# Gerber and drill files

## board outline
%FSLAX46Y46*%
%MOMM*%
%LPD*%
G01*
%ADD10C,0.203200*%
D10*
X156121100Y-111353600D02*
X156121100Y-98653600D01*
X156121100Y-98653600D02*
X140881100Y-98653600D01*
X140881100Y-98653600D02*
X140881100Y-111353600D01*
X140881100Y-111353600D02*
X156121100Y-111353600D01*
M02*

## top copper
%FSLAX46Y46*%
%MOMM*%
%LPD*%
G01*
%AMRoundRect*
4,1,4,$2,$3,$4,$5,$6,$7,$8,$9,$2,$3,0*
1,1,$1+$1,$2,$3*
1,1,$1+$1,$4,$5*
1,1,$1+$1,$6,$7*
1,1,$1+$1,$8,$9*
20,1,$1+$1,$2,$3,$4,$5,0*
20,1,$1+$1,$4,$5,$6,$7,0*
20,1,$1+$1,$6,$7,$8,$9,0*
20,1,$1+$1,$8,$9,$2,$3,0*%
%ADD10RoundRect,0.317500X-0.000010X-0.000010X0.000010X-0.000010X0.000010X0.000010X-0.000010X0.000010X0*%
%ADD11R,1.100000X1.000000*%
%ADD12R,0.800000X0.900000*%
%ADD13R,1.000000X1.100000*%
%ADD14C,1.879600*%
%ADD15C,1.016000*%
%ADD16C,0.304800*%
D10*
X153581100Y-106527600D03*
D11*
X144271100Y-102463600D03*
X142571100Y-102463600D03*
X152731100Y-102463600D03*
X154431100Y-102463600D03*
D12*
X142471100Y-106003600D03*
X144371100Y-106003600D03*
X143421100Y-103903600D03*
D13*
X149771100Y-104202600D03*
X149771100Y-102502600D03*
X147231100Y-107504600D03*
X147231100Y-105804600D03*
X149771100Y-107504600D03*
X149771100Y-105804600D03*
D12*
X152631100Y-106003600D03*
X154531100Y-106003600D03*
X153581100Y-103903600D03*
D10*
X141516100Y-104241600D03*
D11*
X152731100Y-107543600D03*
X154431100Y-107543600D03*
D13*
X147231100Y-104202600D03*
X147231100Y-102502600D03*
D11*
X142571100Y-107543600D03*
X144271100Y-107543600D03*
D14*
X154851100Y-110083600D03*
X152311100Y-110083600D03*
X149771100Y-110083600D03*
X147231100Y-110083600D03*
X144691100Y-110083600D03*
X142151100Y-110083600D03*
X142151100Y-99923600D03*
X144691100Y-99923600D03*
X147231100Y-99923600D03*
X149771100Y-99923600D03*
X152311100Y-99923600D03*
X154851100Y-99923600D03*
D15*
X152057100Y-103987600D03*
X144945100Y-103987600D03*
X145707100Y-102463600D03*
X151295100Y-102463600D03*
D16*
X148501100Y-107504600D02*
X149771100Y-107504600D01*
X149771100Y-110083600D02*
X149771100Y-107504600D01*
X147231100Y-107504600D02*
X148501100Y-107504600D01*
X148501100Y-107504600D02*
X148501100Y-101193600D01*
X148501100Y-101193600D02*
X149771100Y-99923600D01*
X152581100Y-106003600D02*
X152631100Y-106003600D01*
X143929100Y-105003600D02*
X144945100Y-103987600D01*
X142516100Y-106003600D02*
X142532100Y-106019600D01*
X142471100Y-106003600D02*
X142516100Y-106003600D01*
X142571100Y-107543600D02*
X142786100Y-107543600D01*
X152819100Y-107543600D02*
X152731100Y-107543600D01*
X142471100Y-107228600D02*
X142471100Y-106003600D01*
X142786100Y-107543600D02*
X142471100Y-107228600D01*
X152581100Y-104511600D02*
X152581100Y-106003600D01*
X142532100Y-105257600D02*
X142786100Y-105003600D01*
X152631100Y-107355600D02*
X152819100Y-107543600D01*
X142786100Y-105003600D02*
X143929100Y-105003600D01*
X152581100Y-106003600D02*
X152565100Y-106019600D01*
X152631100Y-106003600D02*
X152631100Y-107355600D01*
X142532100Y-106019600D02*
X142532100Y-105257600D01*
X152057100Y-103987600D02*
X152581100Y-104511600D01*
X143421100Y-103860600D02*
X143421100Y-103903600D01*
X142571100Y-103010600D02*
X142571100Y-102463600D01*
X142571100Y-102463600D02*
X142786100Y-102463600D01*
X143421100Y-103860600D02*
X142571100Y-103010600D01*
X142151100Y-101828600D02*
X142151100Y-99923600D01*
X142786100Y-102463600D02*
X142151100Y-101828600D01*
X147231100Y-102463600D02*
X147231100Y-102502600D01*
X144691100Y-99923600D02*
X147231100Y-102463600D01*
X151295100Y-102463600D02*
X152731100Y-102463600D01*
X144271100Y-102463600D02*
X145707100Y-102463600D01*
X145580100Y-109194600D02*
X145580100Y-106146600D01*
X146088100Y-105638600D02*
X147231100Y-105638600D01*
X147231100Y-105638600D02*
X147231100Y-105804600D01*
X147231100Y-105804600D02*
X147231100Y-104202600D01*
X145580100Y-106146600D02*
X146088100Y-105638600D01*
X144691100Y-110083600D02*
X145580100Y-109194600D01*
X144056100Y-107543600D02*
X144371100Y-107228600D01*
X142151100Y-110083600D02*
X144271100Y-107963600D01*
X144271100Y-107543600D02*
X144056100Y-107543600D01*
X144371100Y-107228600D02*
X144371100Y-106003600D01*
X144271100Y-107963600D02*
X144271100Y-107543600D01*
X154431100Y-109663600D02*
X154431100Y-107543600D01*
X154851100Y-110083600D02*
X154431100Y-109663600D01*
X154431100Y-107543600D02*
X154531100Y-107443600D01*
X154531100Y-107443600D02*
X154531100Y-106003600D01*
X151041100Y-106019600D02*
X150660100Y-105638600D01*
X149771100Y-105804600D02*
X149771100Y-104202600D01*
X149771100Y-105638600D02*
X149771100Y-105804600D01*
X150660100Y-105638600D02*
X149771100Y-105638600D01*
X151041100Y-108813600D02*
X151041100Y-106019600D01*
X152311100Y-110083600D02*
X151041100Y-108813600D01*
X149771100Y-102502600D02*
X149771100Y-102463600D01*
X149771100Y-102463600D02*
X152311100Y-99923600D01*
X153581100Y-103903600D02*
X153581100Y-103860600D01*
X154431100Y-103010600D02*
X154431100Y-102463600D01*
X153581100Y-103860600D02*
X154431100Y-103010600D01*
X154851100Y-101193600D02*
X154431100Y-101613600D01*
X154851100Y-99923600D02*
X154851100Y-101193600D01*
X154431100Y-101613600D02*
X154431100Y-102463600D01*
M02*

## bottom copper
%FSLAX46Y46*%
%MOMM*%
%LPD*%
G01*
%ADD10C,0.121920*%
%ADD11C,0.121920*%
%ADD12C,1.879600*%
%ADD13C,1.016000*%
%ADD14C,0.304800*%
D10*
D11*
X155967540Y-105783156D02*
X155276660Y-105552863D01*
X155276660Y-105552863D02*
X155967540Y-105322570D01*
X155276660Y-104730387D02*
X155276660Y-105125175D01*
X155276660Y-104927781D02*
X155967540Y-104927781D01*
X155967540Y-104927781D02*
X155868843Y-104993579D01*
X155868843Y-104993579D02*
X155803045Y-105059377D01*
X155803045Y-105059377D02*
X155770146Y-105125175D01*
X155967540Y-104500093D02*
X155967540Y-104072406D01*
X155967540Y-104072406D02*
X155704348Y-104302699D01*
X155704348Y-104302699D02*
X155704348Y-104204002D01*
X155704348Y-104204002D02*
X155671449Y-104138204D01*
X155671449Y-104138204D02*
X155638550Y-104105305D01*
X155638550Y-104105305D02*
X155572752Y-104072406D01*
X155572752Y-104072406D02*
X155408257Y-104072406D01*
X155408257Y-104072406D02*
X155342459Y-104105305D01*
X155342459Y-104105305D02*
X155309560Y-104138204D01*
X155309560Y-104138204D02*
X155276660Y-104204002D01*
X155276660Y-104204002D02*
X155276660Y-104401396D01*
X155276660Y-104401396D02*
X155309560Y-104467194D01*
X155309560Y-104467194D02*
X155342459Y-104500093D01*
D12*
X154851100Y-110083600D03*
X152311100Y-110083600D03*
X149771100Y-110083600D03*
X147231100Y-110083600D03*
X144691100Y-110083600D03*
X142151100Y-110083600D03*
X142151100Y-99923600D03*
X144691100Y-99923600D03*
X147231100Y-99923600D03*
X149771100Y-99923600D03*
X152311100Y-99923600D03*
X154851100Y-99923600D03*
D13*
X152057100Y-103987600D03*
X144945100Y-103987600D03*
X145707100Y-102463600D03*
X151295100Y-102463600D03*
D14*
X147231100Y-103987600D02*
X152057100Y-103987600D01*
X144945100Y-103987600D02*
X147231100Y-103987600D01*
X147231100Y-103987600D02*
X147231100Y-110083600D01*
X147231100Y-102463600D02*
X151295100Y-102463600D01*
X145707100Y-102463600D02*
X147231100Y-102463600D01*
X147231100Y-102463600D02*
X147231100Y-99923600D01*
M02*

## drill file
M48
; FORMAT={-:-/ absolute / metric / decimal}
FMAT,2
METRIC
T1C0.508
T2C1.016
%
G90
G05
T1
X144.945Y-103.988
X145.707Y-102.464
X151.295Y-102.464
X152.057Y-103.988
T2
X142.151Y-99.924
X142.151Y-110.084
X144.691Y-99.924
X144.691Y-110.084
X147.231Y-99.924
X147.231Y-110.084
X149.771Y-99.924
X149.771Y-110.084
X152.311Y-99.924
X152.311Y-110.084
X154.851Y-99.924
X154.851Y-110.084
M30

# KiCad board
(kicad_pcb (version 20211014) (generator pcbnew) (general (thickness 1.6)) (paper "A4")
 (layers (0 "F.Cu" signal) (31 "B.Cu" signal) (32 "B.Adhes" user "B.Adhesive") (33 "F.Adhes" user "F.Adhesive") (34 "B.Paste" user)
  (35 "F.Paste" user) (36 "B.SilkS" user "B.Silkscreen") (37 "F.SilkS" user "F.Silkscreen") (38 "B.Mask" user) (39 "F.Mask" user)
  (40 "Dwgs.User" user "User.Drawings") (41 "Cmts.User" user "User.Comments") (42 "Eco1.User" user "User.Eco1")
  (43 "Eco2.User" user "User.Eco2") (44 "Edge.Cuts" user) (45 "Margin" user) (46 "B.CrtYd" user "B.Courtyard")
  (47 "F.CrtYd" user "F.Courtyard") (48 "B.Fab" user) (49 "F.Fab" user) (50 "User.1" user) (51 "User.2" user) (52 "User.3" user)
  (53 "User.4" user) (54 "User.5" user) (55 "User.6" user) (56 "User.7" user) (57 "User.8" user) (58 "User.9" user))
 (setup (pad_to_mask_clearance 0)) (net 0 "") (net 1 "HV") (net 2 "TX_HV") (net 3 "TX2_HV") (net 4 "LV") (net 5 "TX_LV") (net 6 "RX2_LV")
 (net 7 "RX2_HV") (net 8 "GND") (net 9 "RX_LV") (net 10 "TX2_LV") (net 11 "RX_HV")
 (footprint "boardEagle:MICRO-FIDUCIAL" (layer "F.Cu") (at 153.5811 106.5276)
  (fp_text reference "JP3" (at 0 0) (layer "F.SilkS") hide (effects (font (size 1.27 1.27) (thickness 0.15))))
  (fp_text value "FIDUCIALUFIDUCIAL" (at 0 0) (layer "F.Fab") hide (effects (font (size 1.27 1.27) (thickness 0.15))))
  (pad "1" smd roundrect (at 0 0) (size 0.635 0.635) (layers "F.Cu" "F.Mask") (roundrect_rratio 0.5) (solder_mask_margin 0.1016)))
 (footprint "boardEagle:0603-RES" (layer "F.Cu") (at 143.4211 102.4636 180)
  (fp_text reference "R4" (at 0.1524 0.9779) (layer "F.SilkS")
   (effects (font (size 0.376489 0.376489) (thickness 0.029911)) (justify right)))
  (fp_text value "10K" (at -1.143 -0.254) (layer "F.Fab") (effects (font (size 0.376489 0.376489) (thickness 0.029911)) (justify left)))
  (pad "1" smd rect (at -0.85 0 180) (size 1.1 1) (layers "F.Cu" "F.Paste" "F.Mask") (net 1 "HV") (solder_mask_margin 0.1016))
  (pad "2" smd rect (at 0.85 0 180) (size 1.1 1) (layers "F.Cu" "F.Paste" "F.Mask") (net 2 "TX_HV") (solder_mask_margin 0.1016)))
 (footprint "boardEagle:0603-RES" (layer "F.Cu") (at 153.5811 102.4636)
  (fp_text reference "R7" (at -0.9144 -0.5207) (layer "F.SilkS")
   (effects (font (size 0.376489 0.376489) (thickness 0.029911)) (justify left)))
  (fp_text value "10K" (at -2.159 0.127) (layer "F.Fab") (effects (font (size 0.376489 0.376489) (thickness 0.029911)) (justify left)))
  (pad "1" smd rect (at -0.85 0) (size 1.1 1) (layers "F.Cu" "F.Paste" "F.Mask") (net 1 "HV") (solder_mask_margin 0.1016))
  (pad "2" smd rect (at 0.85 0) (size 1.1 1) (layers "F.Cu" "F.Paste" "F.Mask") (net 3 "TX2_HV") (solder_mask_margin 0.1016)))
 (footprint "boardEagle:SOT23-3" (layer "F.Cu") (at 143.4211 105.0036)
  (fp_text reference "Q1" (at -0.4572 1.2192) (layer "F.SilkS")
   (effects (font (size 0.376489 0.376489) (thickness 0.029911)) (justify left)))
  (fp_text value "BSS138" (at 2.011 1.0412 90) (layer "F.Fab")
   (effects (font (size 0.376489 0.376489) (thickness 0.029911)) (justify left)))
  (pad "1" smd rect (at -0.95 1) (size 0.8 0.9) (layers "F.Cu" "F.Paste" "F.Mask") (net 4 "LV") (solder_mask_margin 0.1016))
  (pad "2" smd rect (at 0.95 1) (size 0.8 0.9) (layers "F.Cu" "F.Paste" "F.Mask") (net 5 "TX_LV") (solder_mask_margin 0.1016))
  (pad "3" smd rect (at 0 -1.1) (size 0.8 0.9) (layers "F.Cu" "F.Paste" "F.Mask") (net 2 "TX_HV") (solder_mask_margin 0.1016)))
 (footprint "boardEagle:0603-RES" (layer "F.Cu") (at 149.7711 103.3526 90)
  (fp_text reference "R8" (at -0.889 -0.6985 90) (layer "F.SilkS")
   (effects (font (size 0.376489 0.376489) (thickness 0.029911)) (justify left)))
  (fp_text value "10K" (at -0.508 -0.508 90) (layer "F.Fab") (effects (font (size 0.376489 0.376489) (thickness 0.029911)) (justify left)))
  (pad "1" smd rect (at -0.85 0 90) (size 1.1 1) (layers "F.Cu" "F.Paste" "F.Mask") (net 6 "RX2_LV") (solder_mask_margin 0.1016))
  (pad "2" smd rect (at 0.85 0 90) (size 1.1 1) (layers "F.Cu" "F.Paste" "F.Mask") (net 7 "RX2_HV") (solder_mask_margin 0.1016)))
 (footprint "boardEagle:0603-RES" (layer "F.Cu") (at 147.2311 106.6546 90)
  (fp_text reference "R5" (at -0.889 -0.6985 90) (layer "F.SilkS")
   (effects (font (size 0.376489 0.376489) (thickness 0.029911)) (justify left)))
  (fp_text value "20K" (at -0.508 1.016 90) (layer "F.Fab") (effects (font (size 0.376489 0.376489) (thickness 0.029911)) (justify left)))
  (pad "1" smd rect (at -0.85 0 90) (size 1.1 1) (layers "F.Cu" "F.Paste" "F.Mask") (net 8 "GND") (solder_mask_margin 0.1016))
  (pad "2" smd rect (at 0.85 0 90) (size 1.1 1) (layers "F.Cu" "F.Paste" "F.Mask") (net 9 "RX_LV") (solder_mask_margin 0.1016)))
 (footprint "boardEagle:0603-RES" (layer "F.Cu") (at 149.7711 106.6546 90)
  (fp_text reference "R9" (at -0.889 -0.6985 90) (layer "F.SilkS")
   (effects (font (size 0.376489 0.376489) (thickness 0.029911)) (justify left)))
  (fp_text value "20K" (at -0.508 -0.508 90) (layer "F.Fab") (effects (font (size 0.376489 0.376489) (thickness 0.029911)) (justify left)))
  (pad "1" smd rect (at -0.85 0 90) (size 1.1 1) (layers "F.Cu" "F.Paste" "F.Mask") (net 8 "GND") (solder_mask_margin 0.1016))
  (pad "2" smd rect (at 0.85 0 90) (size 1.1 1) (layers "F.Cu" "F.Paste" "F.Mask") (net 6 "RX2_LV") (solder_mask_margin 0.1016)))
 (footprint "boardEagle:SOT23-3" (layer "F.Cu") (at 153.5811 105.0036)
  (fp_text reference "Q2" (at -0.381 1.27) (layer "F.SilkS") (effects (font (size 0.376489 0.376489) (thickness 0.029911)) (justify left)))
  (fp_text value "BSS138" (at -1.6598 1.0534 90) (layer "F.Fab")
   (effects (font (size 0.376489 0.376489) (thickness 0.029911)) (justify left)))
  (pad "1" smd rect (at -0.95 1) (size 0.8 0.9) (layers "F.Cu" "F.Paste" "F.Mask") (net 4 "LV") (solder_mask_margin 0.1016))
  (pad "2" smd rect (at 0.95 1) (size 0.8 0.9) (layers "F.Cu" "F.Paste" "F.Mask") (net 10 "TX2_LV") (solder_mask_margin 0.1016))
  (pad "3" smd rect (at 0 -1.1) (size 0.8 0.9) (layers "F.Cu" "F.Paste" "F.Mask") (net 3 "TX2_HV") (solder_mask_margin 0.1016)))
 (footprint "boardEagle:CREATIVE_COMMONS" (layer "F.Cu") (at 162.4711 118.9736)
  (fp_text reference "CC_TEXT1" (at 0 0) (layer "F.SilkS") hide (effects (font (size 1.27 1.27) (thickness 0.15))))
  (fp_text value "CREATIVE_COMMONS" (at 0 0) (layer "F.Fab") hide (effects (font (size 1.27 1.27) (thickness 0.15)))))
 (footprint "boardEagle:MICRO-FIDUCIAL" (layer "F.Cu") (at 141.5161 104.2416)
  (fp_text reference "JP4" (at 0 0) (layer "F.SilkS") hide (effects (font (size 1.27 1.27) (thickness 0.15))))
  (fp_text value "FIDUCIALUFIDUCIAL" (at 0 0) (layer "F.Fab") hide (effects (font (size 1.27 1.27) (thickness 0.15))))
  (pad "1" smd roundrect (at 0 0) (size 0.635 0.635) (layers "F.Cu" "F.Mask") (roundrect_rratio 0.5) (solder_mask_margin 0.1016)))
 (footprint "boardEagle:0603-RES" (layer "F.Cu") (at 153.5811 107.5436)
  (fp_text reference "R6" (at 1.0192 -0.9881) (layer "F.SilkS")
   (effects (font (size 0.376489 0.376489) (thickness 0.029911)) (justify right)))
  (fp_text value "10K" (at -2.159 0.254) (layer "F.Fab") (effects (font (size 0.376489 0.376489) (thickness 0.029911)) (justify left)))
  (pad "1" smd rect (at -0.85 0) (size 1.1 1) (layers "F.Cu" "F.Paste" "F.Mask") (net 4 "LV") (solder_mask_margin 0.1016))
  (pad "2" smd rect (at 0.85 0) (size 1.1 1) (layers "F.Cu" "F.Paste" "F.Mask") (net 10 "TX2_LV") (solder_mask_margin 0.1016)))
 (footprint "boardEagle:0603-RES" (layer "F.Cu") (at 147.2311 103.3526 90)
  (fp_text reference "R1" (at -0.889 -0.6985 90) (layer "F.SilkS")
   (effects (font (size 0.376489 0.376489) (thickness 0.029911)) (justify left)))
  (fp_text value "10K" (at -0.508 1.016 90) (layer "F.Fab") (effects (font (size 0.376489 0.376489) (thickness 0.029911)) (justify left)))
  (pad "1" smd rect (at -0.85 0 90) (size 1.1 1) (layers "F.Cu" "F.Paste" "F.Mask") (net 9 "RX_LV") (solder_mask_margin 0.1016))
  (pad "2" smd rect (at 0.85 0 90) (size 1.1 1) (layers "F.Cu" "F.Paste" "F.Mask") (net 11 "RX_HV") (solder_mask_margin 0.1016)))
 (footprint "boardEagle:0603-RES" (layer "F.Cu") (at 143.4211 107.5436)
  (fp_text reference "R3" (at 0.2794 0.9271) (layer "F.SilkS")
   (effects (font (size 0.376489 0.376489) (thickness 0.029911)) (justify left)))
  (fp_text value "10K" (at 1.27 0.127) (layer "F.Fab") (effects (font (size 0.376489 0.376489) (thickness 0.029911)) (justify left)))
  (pad "1" smd rect (at -0.85 0) (size 1.1 1) (layers "F.Cu" "F.Paste" "F.Mask") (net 4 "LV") (solder_mask_margin 0.1016))
  (pad "2" smd rect (at 0.85 0) (size 1.1 1) (layers "F.Cu" "F.Paste" "F.Mask") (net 5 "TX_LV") (solder_mask_margin 0.1016)))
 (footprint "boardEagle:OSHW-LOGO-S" (layer "B.Cu") (at 142.6591 102.9716 180)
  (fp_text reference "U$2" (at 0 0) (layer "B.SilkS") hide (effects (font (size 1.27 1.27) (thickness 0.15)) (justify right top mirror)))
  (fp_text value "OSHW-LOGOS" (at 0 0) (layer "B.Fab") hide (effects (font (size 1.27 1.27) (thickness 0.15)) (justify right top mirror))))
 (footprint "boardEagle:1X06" (layer "B.Cu") (at 154.8511 110.0836 180)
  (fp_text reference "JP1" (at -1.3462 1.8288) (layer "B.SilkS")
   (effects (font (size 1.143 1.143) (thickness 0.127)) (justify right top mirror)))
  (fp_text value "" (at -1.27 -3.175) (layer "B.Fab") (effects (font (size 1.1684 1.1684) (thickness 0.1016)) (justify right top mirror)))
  (pad "1" thru_hole circle (at 0 0 90) (size 1.8796 1.8796) (drill 1.016) (layers *.Cu *.Mask) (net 10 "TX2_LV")
   (solder_mask_margin 0.1016))
  (pad "2" thru_hole circle (at 2.54 0 90) (size 1.8796 1.8796) (drill 1.016) (layers *.Cu *.Mask) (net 6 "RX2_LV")
   (solder_mask_margin 0.1016))
  (pad "3" thru_hole circle (at 5.08 0 90) (size 1.8796 1.8796) (drill 1.016) (layers *.Cu *.Mask) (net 8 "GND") (solder_mask_margin 0.1016))
  (pad "4" thru_hole circle (at 7.62 0 90) (size 1.8796 1.8796) (drill 1.016) (layers *.Cu *.Mask) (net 4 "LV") (solder_mask_margin 0.1016))
  (pad "5" thru_hole circle (at 10.16 0 90) (size 1.8796 1.8796) (drill 1.016) (layers *.Cu *.Mask) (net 9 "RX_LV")
   (solder_mask_margin 0.1016))
  (pad "6" thru_hole circle (at 12.7 0 90) (size 1.8796 1.8796) (drill 1.016) (layers *.Cu *.Mask) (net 5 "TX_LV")
   (solder_mask_margin 0.1016)))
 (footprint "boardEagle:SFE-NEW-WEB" (layer "B.Cu") (at 154.7241 106.9086 180)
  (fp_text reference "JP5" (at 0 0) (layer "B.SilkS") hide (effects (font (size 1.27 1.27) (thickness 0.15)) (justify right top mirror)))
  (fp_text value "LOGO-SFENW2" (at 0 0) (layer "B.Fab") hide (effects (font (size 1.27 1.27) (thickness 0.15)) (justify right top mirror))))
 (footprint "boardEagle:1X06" (layer "B.Cu") (at 142.1511 99.9236)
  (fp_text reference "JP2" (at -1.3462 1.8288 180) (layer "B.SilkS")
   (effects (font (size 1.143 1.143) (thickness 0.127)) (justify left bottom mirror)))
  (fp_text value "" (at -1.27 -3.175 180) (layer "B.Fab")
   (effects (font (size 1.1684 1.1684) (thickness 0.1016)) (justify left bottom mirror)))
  (pad "1" thru_hole circle (at 0 0 270) (size 1.8796 1.8796) (drill 1.016) (layers *.Cu *.Mask) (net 2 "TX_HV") (solder_mask_margin 0.1016))
  (pad "2" thru_hole circle (at 2.54 0 270) (size 1.8796 1.8796) (drill 1.016) (layers *.Cu *.Mask) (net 11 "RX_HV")
   (solder_mask_margin 0.1016))
  (pad "3" thru_hole circle (at 5.08 0 270) (size 1.8796 1.8796) (drill 1.016) (layers *.Cu *.Mask) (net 1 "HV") (solder_mask_margin 0.1016))
  (pad "4" thru_hole circle (at 7.62 0 270) (size 1.8796 1.8796) (drill 1.016) (layers *.Cu *.Mask) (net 8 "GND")
   (solder_mask_margin 0.1016))
  (pad "5" thru_hole circle (at 10.16 0 270) (size 1.8796 1.8796) (drill 1.016) (layers *.Cu *.Mask) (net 7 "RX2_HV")
   (solder_mask_margin 0.1016))
  (pad "6" thru_hole circle (at 12.7 0 270) (size 1.8796 1.8796) (drill 1.016) (layers *.Cu *.Mask) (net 3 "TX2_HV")
   (solder_mask_margin 0.1016)))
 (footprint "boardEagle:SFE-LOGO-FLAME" (layer "B.Cu") (at 147.6121 104.2416 180)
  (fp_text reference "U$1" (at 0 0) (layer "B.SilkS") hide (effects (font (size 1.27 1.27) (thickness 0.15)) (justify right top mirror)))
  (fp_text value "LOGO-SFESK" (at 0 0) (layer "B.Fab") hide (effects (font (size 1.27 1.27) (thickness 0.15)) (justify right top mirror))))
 (gr_line (start 156.1211 111.3536) (end 156.1211 98.6536) (layer "Edge.Cuts") (width 0.2032))
 (gr_line (start 156.1211 98.6536) (end 140.8811 98.6536) (layer "Edge.Cuts") (width 0.2032))
 (gr_line (start 140.8811 98.6536) (end 140.8811 111.3536) (layer "Edge.Cuts") (width 0.2032))
 (gr_line (start 140.8811 111.3536) (end 156.1211 111.3536) (layer "Edge.Cuts") (width 0.2032))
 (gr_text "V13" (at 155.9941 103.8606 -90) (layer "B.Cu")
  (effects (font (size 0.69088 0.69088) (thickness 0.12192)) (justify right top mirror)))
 (segment (start 148.5011 107.5046) (end 149.7711 107.5046) (width 0.3048) (layer "F.Cu") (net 8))
 (segment (start 149.7711 110.0836) (end 149.7711 107.5046) (width 0.3048) (layer "F.Cu") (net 8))
 (segment (start 147.2311 107.5046) (end 148.5011 107.5046) (width 0.3048) (layer "F.Cu") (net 8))
 (segment (start 148.5011 107.5046) (end 148.5011 101.1936) (width 0.3048) (layer "F.Cu") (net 8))
 (segment (start 148.5011 101.1936) (end 149.7711 99.9236) (width 0.3048) (layer "F.Cu") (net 8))
 (segment (start 152.5811 106.0036) (end 152.6311 106.0036) (width 0.3048) (layer "F.Cu") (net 4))
 (segment (start 143.9291 105.0036) (end 144.9451 103.9876) (width 0.3048) (layer "F.Cu") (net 4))
 (segment (start 142.5161 106.0036) (end 142.5321 106.0196) (width 0.3048) (layer "F.Cu") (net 4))
 (segment (start 142.4711 106.0036) (end 142.5161 106.0036) (width 0.3048) (layer "F.Cu") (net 4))
 (segment (start 142.5711 107.5436) (end 142.7861 107.5436) (width 0.3048) (layer "F.Cu") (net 4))
 (segment (start 152.8191 107.5436) (end 152.7311 107.5436) (width 0.3048) (layer "F.Cu") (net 4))
 (segment (start 142.4711 107.2286) (end 142.4711 106.0036) (width 0.3048) (layer "F.Cu") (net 4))
 (segment (start 142.7861 107.5436) (end 142.4711 107.2286) (width 0.3048) (layer "F.Cu") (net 4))
 (segment (start 152.5811 104.5116) (end 152.5811 106.0036) (width 0.3048) (layer "F.Cu") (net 4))
 (segment (start 142.5321 105.2576) (end 142.7861 105.0036) (width 0.3048) (layer "F.Cu") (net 4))
 (segment (start 152.6311 107.3556) (end 152.8191 107.5436) (width 0.3048) (layer "F.Cu") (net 4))
 (segment (start 142.7861 105.0036) (end 143.9291 105.0036) (width 0.3048) (layer "F.Cu") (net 4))
 (segment (start 152.5811 106.0036) (end 152.5651 106.0196) (width 0.3048) (layer "F.Cu") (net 4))
 (segment (start 152.6311 106.0036) (end 152.6311 107.3556) (width 0.3048) (layer "F.Cu") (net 4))
 (segment (start 142.5321 106.0196) (end 142.5321 105.2576) (width 0.3048) (layer "F.Cu") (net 4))
 (segment (start 152.0571 103.9876) (end 152.5811 104.5116) (width 0.3048) (layer "F.Cu") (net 4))
 (via (at 152.0571 103.9876) (size 1.016) (drill 0.508) (layers "F.Cu" "B.Cu") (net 4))
 (via (at 144.9451 103.9876) (size 1.016) (drill 0.508) (layers "F.Cu" "B.Cu") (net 4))
 (segment (start 147.2311 103.9876) (end 152.0571 103.9876) (width 0.3048) (layer "B.Cu") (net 4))
 (segment (start 144.9451 103.9876) (end 147.2311 103.9876) (width 0.3048) (layer "B.Cu") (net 4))
 (segment (start 147.2311 103.9876) (end 147.2311 110.0836) (width 0.3048) (layer "B.Cu") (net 4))
 (segment (start 143.4211 103.8606) (end 143.4211 103.9036) (width 0.3048) (layer "F.Cu") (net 2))
 (segment (start 142.5711 103.0106) (end 142.5711 102.4636) (width 0.3048) (layer "F.Cu") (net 2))
 (segment (start 142.5711 102.4636) (end 142.7861 102.4636) (width 0.3048) (layer "F.Cu") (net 2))
 (segment (start 143.4211 103.8606) (end 142.5711 103.0106) (width 0.3048) (layer "F.Cu") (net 2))
 (segment (start 142.1511 101.8286) (end 142.1511 99.9236) (width 0.3048) (layer "F.Cu") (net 2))
 (segment (start 142.7861 102.4636) (end 142.1511 101.8286) (width 0.3048) (layer "F.Cu") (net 2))
 (segment (start 147.2311 102.4636) (end 147.2311 102.5026) (width 0.3048) (layer "F.Cu") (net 11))
 (segment (start 144.6911 99.9236) (end 147.2311 102.4636) (width 0.3048) (layer "F.Cu") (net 11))
 (segment (start 151.2951 102.4636) (end 152.7311 102.4636) (width 0.3048) (layer "F.Cu") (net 1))
 (segment (start 144.2711 102.4636) (end 145.7071 102.4636) (width 0.3048) (layer "F.Cu") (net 1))
 (via (at 145.7071 102.4636) (size 1.016) (drill 0.508) (layers "F.Cu" "B.Cu") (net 1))
 (via (at 151.2951 102.4636) (size 1.016) (drill 0.508) (layers "F.Cu" "B.Cu") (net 1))
 (segment (start 147.2311 102.4636) (end 151.2951 102.4636) (width 0.3048) (layer "B.Cu") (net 1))
 (segment (start 145.7071 102.4636) (end 147.2311 102.4636) (width 0.3048) (layer "B.Cu") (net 1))
 (segment (start 147.2311 102.4636) (end 147.2311 99.9236) (width 0.3048) (layer "B.Cu") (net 1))
 (segment (start 145.5801 109.1946) (end 145.5801 106.1466) (width 0.3048) (layer "F.Cu") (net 9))
 (segment (start 146.0881 105.6386) (end 147.2311 105.6386) (width 0.3048) (layer "F.Cu") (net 9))
 (segment (start 147.2311 105.6386) (end 147.2311 105.8046) (width 0.3048) (layer "F.Cu") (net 9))
 (segment (start 147.2311 105.8046) (end 147.2311 104.2026) (width 0.3048) (layer "F.Cu") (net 9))
 (segment (start 145.5801 106.1466) (end 146.0881 105.6386) (width 0.3048) (layer "F.Cu") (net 9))
 (segment (start 144.6911 110.0836) (end 145.5801 109.1946) (width 0.3048) (layer "F.Cu") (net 9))
 (segment (start 144.0561 107.5436) (end 144.3711 107.2286) (width 0.3048) (layer "F.Cu") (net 5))
 (segment (start 142.1511 110.0836) (end 144.2711 107.9636) (width 0.3048) (layer "F.Cu") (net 5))
 (segment (start 144.2711 107.5436) (end 144.0561 107.5436) (width 0.3048) (layer "F.Cu") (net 5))
 (segment (start 144.3711 107.2286) (end 144.3711 106.0036) (width 0.3048) (layer "F.Cu") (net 5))
 (segment (start 144.2711 107.9636) (end 144.2711 107.5436) (width 0.3048) (layer "F.Cu") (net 5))
 (segment (start 154.4311 109.6636) (end 154.4311 107.5436) (width 0.3048) (layer "F.Cu") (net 10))
 (segment (start 154.8511 110.0836) (end 154.4311 109.6636) (width 0.3048) (layer "F.Cu") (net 10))
 (segment (start 154.4311 107.5436) (end 154.5311 107.4436) (width 0.3048) (layer "F.Cu") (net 10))
 (segment (start 154.5311 107.4436) (end 154.5311 106.0036) (width 0.3048) (layer "F.Cu") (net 10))
 (segment (start 151.0411 106.0196) (end 150.6601 105.6386) (width 0.3048) (layer "F.Cu") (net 6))
 (segment (start 149.7711 105.8046) (end 149.7711 104.2026) (width 0.3048) (layer "F.Cu") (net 6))
 (segment (start 149.7711 105.6386) (end 149.7711 105.8046) (width 0.3048) (layer "F.Cu") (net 6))
 (segment (start 150.6601 105.6386) (end 149.7711 105.6386) (width 0.3048) (layer "F.Cu") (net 6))
 (segment (start 151.0411 108.8136) (end 151.0411 106.0196) (width 0.3048) (layer "F.Cu") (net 6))
 (segment (start 152.3111 110.0836) (end 151.0411 108.8136) (width 0.3048) (layer "F.Cu") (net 6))
 (segment (start 149.7711 102.5026) (end 149.7711 102.4636) (width 0.3048) (layer "F.Cu") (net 7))
 (segment (start 149.7711 102.4636) (end 152.3111 99.9236) (width 0.3048) (layer "F.Cu") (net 7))
 (segment (start 153.5811 103.9036) (end 153.5811 103.8606) (width 0.3048) (layer "F.Cu") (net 3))
 (segment (start 154.4311 103.0106) (end 154.4311 102.4636) (width 0.3048) (layer "F.Cu") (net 3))
 (segment (start 153.5811 103.8606) (end 154.4311 103.0106) (width 0.3048) (layer "F.Cu") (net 3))
 (segment (start 154.8511 101.1936) (end 154.4311 101.6136) (width 0.3048) (layer "F.Cu") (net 3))
 (segment (start 154.8511 99.9236) (end 154.8511 101.1936) (width 0.3048) (layer "F.Cu") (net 3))
 (segment (start 154.4311 101.6136) (end 154.4311 102.4636) (width 0.3048) (layer "F.Cu") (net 3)))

